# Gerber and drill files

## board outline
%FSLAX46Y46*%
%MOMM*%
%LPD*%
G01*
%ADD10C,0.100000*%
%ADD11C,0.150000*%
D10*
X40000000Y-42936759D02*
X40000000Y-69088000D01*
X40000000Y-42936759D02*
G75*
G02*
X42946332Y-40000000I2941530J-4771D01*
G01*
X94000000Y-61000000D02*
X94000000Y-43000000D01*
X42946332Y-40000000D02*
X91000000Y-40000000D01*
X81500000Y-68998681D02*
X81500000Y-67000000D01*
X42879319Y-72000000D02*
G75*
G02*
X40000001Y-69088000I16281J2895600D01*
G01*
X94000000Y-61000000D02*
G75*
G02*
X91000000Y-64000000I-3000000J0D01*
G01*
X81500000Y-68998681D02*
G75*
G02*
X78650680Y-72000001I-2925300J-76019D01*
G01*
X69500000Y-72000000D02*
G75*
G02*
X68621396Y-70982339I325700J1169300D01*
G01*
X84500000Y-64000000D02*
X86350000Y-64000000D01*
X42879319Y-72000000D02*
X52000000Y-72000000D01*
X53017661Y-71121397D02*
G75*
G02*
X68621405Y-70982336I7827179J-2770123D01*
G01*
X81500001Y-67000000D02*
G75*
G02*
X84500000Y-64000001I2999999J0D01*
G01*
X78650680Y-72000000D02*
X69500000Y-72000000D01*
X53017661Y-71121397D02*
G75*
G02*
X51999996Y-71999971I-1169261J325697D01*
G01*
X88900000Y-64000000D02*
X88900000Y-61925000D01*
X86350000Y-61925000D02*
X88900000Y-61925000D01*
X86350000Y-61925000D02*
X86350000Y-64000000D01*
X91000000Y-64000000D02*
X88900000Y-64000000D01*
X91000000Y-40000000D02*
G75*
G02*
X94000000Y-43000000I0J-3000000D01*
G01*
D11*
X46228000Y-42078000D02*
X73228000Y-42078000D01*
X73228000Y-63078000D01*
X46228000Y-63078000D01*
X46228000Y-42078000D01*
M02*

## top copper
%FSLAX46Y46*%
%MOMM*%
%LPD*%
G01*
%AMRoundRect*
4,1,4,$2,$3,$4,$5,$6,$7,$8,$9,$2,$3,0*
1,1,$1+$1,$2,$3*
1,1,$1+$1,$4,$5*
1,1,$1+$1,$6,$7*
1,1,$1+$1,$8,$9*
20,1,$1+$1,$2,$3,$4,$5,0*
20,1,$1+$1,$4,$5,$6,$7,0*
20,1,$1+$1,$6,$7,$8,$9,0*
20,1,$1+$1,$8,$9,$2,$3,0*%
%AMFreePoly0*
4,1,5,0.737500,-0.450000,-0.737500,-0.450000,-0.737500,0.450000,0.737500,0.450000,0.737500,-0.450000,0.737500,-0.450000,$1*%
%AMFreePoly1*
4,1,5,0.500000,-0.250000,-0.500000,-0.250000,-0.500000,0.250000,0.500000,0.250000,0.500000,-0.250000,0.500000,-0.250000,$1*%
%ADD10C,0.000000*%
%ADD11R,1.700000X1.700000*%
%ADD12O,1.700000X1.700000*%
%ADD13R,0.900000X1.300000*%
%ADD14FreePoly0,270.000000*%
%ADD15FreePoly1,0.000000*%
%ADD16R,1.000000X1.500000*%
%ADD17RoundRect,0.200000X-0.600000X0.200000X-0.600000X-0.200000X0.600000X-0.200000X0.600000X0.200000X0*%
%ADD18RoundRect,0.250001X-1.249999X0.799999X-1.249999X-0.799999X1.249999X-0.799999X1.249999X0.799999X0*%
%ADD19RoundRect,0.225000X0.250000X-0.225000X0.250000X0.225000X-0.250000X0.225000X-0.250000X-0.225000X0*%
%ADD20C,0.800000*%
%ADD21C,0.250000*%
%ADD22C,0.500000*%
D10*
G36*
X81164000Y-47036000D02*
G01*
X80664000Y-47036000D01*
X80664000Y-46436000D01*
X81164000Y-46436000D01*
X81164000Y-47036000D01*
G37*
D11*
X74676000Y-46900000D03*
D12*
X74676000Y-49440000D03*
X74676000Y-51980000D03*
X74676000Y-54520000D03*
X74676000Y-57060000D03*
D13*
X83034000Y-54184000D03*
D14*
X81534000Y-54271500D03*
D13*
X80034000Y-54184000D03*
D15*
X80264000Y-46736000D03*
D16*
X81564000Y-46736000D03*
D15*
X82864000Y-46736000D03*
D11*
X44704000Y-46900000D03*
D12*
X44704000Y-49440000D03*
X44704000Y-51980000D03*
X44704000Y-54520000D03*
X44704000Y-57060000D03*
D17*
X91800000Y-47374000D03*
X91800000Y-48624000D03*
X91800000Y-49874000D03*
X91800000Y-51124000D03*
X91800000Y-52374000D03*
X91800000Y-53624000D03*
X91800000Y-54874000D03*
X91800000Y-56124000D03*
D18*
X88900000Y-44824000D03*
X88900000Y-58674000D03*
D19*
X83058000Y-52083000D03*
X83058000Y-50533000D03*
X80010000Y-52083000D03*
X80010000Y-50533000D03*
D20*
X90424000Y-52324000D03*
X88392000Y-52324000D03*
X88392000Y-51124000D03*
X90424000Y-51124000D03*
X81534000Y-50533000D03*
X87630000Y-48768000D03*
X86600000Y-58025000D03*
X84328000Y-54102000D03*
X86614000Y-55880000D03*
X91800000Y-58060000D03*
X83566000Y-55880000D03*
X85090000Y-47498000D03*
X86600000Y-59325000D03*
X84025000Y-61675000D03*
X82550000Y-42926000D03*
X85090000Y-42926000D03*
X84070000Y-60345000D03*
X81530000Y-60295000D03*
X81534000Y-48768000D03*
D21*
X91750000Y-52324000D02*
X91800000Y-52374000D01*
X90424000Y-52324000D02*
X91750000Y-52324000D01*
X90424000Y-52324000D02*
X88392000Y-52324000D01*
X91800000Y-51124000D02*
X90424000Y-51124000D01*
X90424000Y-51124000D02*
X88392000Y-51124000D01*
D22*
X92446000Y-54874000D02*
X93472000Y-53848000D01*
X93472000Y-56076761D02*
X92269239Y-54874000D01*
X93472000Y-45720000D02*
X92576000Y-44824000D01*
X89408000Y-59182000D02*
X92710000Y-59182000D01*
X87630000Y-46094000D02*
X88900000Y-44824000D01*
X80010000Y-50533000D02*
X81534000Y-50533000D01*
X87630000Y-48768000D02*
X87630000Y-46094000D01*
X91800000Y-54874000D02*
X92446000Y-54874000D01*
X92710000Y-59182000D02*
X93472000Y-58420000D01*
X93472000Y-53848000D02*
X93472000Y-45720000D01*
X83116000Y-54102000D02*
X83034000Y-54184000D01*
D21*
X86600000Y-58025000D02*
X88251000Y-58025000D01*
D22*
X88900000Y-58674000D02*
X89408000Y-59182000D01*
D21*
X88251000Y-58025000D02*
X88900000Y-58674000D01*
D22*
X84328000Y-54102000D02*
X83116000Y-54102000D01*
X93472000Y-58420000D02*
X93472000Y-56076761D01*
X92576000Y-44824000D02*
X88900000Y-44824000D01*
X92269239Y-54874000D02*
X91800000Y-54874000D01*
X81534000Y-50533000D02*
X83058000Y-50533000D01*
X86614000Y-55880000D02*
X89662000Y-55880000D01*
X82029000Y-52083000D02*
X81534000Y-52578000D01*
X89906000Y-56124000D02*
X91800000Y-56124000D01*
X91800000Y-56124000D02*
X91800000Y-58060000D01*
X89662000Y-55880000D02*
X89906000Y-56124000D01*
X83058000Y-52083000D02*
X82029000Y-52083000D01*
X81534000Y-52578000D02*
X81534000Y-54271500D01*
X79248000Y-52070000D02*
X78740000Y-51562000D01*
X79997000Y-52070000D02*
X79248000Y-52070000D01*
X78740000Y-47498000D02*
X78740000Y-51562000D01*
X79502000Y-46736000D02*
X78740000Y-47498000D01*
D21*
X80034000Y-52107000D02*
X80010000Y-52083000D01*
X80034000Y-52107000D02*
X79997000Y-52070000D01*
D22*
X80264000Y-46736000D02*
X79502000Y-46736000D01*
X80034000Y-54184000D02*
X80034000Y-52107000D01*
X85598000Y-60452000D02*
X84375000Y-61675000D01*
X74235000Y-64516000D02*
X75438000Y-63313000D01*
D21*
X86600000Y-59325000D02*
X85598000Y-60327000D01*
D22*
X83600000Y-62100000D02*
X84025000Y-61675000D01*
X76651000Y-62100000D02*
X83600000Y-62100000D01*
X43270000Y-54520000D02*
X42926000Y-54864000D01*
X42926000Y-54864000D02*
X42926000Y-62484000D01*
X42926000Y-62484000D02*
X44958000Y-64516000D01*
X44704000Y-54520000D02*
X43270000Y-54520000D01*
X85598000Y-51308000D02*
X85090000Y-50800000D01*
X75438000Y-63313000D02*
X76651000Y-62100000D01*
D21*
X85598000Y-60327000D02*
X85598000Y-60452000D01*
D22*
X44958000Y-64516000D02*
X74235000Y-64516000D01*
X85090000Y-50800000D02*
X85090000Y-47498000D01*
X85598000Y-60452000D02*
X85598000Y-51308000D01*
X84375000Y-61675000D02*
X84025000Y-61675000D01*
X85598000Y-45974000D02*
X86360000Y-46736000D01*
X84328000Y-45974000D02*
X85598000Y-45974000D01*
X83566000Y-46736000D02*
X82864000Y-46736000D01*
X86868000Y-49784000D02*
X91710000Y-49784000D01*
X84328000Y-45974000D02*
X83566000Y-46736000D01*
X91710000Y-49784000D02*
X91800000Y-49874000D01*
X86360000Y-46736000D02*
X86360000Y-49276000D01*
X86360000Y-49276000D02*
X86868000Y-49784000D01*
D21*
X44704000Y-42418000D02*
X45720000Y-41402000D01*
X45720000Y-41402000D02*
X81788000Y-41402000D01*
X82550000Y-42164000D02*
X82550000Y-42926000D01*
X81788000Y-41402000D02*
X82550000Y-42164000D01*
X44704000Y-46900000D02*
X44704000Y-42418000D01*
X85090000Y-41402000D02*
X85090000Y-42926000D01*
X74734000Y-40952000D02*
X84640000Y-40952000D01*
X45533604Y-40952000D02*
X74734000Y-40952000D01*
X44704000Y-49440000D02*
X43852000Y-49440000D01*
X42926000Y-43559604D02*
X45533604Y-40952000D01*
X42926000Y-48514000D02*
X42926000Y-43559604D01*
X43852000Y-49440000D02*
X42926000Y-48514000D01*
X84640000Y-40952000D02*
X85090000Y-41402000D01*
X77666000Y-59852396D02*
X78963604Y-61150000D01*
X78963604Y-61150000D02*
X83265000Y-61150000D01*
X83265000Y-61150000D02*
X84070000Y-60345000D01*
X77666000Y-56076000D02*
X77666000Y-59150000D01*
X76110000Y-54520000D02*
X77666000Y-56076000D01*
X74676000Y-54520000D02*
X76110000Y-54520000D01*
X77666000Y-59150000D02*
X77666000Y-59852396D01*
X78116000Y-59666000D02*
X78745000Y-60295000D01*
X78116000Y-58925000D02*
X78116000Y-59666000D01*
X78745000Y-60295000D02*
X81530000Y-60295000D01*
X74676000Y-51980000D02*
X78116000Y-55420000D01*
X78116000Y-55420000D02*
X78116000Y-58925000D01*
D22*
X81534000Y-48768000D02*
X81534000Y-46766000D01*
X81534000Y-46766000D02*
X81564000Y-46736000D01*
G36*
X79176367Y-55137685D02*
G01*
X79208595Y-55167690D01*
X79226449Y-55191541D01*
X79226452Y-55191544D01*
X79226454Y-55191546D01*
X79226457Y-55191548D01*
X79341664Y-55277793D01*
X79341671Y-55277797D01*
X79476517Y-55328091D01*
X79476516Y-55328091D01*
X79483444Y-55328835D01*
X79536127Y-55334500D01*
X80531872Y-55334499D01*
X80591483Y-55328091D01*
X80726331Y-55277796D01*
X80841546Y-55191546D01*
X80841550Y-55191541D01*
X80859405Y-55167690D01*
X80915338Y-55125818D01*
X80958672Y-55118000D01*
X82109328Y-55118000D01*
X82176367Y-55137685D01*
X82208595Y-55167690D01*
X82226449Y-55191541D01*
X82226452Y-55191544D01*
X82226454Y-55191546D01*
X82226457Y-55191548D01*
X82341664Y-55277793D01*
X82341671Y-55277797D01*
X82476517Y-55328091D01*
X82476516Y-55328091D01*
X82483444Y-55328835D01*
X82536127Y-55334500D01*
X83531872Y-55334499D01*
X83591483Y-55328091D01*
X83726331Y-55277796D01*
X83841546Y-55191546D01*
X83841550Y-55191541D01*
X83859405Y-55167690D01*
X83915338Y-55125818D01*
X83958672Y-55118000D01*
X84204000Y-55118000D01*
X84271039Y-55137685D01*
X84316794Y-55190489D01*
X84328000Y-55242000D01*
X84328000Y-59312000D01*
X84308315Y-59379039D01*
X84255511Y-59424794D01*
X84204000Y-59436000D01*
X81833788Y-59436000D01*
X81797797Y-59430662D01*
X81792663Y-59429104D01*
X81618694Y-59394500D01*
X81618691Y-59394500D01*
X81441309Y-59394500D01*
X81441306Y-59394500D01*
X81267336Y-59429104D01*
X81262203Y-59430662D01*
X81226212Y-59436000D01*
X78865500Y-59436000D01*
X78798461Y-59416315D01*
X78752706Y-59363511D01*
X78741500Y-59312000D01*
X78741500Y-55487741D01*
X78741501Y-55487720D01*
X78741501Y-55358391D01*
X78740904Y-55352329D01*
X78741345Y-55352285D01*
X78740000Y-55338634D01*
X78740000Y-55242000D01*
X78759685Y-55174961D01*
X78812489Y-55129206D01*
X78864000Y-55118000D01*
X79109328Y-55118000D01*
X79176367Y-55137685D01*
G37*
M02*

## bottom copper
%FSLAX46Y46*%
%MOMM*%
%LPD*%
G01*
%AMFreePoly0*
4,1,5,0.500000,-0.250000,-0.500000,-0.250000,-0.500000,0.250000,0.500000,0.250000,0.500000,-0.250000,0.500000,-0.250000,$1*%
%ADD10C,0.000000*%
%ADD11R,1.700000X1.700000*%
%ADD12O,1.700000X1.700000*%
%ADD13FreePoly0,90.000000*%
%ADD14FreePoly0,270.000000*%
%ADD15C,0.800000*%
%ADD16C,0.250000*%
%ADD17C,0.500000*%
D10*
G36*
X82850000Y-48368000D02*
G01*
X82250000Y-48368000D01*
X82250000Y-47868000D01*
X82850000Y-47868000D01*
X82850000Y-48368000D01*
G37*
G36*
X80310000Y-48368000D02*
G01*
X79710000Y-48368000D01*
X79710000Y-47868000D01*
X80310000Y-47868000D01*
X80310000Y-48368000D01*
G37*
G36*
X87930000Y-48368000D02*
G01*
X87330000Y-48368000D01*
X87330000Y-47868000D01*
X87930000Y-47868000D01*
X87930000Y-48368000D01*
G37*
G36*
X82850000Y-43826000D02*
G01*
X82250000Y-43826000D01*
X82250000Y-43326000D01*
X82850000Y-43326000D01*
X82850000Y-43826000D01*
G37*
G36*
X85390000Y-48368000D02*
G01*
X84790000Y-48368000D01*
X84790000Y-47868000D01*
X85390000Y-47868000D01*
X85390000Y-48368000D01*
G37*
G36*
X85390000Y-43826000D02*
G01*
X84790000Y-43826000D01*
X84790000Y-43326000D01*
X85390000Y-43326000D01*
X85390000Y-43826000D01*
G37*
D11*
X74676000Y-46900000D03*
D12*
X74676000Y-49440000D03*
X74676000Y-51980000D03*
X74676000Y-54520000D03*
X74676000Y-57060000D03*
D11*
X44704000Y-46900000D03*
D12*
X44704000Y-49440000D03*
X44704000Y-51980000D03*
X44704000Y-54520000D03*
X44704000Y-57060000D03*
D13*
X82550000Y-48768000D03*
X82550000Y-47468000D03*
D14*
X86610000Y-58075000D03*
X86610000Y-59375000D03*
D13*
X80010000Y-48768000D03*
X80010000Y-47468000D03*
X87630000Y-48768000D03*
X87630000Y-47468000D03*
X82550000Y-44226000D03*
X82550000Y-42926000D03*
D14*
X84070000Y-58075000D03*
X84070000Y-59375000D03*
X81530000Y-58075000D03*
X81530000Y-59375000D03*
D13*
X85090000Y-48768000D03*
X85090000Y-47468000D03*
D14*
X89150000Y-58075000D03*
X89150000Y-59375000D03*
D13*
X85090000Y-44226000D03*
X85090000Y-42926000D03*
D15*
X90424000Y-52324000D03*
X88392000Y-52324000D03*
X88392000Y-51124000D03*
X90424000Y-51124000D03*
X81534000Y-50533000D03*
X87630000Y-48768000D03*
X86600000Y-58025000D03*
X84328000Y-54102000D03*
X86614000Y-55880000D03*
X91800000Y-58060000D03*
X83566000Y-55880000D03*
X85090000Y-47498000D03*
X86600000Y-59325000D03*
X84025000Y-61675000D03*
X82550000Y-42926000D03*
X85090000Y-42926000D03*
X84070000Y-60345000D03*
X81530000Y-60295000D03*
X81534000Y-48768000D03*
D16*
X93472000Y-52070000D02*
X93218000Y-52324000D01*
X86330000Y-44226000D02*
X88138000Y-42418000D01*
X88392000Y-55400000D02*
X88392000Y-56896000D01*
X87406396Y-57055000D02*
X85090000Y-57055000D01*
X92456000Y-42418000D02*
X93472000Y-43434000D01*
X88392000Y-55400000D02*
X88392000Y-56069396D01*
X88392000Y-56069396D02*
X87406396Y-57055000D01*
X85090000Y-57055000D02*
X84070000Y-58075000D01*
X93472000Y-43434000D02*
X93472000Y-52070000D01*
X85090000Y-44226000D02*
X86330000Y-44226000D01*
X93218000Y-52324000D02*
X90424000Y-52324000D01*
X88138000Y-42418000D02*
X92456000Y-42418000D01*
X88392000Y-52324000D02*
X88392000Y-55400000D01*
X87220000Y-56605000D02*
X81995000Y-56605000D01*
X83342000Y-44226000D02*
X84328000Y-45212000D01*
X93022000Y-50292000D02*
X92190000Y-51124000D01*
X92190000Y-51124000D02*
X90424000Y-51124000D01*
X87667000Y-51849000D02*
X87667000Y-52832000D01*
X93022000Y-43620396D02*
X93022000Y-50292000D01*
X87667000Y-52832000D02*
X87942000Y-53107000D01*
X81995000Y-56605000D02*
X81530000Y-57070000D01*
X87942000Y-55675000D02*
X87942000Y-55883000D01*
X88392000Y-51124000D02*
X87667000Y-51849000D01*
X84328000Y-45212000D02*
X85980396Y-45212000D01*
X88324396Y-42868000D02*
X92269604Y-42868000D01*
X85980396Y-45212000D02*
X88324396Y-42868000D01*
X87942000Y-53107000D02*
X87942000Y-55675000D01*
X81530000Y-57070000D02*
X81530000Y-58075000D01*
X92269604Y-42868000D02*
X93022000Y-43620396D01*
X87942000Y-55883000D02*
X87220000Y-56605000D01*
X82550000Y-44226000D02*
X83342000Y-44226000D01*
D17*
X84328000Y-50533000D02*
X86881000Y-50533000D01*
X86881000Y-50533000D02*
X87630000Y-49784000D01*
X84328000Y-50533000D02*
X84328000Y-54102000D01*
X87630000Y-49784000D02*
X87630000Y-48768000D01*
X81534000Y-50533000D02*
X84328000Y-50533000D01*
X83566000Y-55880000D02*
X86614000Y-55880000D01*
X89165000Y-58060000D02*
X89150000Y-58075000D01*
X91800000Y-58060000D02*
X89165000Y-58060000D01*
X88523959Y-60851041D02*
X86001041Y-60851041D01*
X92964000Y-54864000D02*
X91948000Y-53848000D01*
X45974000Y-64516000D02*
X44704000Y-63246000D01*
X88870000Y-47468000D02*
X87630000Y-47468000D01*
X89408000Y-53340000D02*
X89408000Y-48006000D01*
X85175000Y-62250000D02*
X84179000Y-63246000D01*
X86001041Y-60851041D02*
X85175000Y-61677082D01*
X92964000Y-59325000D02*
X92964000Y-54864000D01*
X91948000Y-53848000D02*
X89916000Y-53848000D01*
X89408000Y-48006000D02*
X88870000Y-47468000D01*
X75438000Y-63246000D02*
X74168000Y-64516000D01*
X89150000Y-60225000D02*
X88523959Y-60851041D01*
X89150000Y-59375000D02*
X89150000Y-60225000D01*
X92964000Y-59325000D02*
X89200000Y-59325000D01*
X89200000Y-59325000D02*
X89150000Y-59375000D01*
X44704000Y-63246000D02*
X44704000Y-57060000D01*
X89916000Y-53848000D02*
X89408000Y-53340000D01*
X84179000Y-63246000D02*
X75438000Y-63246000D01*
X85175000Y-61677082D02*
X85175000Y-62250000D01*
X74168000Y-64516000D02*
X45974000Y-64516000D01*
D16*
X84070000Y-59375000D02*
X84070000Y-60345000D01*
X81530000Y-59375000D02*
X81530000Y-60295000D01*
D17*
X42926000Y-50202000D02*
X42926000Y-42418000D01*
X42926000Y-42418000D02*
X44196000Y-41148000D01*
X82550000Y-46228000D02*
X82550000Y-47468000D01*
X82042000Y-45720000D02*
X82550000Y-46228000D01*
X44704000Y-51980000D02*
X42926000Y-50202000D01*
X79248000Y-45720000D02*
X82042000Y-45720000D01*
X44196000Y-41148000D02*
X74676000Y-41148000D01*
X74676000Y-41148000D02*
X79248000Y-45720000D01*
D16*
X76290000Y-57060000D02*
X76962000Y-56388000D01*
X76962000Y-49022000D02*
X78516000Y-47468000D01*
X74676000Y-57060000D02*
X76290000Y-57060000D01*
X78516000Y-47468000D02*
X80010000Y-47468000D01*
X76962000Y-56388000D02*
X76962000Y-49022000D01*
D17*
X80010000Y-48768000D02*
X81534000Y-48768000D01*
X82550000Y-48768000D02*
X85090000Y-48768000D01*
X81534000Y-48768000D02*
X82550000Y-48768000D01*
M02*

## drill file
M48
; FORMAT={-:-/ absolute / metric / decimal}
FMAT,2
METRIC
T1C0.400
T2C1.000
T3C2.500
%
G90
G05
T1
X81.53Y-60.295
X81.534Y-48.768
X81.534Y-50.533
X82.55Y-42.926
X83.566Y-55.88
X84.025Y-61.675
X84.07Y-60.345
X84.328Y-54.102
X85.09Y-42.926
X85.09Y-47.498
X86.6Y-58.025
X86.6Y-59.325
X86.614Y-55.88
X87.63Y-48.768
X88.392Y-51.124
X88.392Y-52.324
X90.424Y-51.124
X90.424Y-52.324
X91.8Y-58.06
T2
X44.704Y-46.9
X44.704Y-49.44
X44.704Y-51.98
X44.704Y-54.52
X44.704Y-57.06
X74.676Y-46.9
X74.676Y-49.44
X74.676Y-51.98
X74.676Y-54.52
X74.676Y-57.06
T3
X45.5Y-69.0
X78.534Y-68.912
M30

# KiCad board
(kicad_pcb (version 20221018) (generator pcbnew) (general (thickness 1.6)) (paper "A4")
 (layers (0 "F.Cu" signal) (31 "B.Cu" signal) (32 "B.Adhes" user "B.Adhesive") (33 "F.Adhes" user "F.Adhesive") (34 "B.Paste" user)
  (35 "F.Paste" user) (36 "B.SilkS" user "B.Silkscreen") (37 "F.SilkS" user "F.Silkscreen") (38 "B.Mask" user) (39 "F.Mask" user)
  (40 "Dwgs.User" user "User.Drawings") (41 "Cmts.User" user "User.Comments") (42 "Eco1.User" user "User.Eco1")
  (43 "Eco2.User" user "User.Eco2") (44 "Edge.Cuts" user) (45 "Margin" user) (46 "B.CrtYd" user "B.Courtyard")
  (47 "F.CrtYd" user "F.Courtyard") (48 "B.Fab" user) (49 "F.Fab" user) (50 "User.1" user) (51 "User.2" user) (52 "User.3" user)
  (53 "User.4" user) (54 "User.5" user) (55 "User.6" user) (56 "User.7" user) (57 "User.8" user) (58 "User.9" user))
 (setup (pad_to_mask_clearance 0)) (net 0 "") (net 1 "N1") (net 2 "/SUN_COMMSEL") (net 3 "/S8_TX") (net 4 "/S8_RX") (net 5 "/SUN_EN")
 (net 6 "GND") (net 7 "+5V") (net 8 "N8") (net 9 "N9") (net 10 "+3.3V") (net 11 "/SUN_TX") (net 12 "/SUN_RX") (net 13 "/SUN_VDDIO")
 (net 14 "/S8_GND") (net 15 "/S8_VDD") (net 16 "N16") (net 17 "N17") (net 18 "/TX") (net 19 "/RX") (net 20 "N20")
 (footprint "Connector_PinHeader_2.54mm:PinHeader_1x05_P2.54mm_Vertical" (layer "F.Cu") (at 74.676 46.9)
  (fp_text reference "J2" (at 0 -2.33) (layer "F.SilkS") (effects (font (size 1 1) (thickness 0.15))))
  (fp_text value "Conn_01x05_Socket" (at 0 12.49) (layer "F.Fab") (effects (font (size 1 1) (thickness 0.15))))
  (pad "1" thru_hole rect (at 0 0) (size 1.7 1.7) (drill 1) (layers "*.Cu" "*.Mask") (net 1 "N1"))
  (pad "2" thru_hole oval (at 0 2.54) (size 1.7 1.7) (drill 1) (layers "*.Cu" "*.Mask") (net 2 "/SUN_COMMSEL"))
  (pad "3" thru_hole oval (at 0 5.08) (size 1.7 1.7) (drill 1) (layers "*.Cu" "*.Mask") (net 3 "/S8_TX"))
  (pad "4" thru_hole oval (at 0 7.62) (size 1.7 1.7) (drill 1) (layers "*.Cu" "*.Mask") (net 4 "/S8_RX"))
  (pad "5" thru_hole oval (at 0 10.16) (size 1.7 1.7) (drill 1) (layers "*.Cu" "*.Mask") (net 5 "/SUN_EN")))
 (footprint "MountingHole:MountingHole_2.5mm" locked (layer "F.Cu") (at 45.466 69.088)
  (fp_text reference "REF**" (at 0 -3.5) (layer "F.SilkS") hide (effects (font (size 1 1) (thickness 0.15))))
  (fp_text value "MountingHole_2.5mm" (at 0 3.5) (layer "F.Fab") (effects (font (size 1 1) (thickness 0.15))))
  (pad "" np_thru_hole circle locked (at 0.034 -0.088) (size 2.5 2.5) (drill 2.5) (layers "F&B.Cu" "*.Mask")))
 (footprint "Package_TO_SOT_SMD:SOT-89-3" (layer "F.Cu") (at 81.534 56.134 -90)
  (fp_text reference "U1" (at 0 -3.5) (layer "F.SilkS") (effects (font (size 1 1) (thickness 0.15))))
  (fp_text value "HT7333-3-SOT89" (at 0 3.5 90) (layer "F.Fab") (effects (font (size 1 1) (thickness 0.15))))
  (pad "1" smd rect (at -1.95 -1.5 270) (size 1.3 0.9) (layers "F.Cu" "F.Paste" "F.Mask") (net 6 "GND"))
  (pad "2" smd custom (at -1.8625 0 270) (size 1.475 0.9) (layers "F.Cu" "F.Paste" "F.Mask") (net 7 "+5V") (zone_connect 2)
   (thermal_bridge_angle 45) (options (clearance outline) (anchor rect)) (primitives))
  (pad "3" smd rect (at -1.95 1.5 270) (size 1.3 0.9) (layers "F.Cu" "F.Paste" "F.Mask") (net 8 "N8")))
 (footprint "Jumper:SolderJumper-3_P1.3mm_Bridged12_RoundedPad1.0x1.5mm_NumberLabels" (layer "F.Cu") (at 81.564 46.736)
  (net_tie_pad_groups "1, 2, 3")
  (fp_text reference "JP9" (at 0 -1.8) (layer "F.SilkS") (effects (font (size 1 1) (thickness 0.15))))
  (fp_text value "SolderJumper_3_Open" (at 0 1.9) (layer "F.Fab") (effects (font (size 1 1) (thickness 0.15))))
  (fp_poly (pts (xy -0.9 -0.3) (xy -0.4 -0.3) (xy -0.4 0.3) (xy -0.9 0.3)) (stroke (width 0) (type solid)) (fill solid) (layer "F.Cu"))
  (pad "1" smd custom (at -1.3 0) (size 1 0.5) (layers "F.Cu" "F.Mask") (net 8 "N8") (zone_connect 2) (thermal_bridge_angle 45)
   (options (clearance outline) (anchor rect)) (primitives))
  (pad "2" smd rect (at 0 0) (size 1 1.5) (layers "F.Cu" "F.Mask") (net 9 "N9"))
  (pad "3" smd custom (at 1.3 0) (size 1 0.5) (layers "F.Cu" "F.Mask") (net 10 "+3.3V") (zone_connect 2) (thermal_bridge_angle 45)
   (options (clearance outline) (anchor rect)) (primitives)))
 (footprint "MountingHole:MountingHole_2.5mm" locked (layer "F.Cu") (at 78.5 69)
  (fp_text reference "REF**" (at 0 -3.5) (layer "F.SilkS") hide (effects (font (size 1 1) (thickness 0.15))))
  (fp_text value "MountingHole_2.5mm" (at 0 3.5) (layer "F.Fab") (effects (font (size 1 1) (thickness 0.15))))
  (pad "" np_thru_hole circle locked (at 0.034 -0.088) (size 2.5 2.5) (drill 2.5) (layers "F&B.Cu" "*.Mask")))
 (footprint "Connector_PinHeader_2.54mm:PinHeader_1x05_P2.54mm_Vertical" (layer "F.Cu") (at 44.704 46.9)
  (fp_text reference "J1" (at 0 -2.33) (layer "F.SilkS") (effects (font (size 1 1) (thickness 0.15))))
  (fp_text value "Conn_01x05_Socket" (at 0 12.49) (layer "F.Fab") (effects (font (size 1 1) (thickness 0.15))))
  (pad "1" thru_hole rect (at 0 0) (size 1.7 1.7) (drill 1) (layers "*.Cu" "*.Mask") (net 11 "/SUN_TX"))
  (pad "2" thru_hole oval (at 0 2.54) (size 1.7 1.7) (drill 1) (layers "*.Cu" "*.Mask") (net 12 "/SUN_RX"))
  (pad "3" thru_hole oval (at 0 5.08) (size 1.7 1.7) (drill 1) (layers "*.Cu" "*.Mask") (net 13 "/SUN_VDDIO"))
  (pad "4" thru_hole oval (at 0 7.62) (size 1.7 1.7) (drill 1) (layers "*.Cu" "*.Mask") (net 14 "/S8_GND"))
  (pad "5" thru_hole oval (at 0 10.16) (size 1.7 1.7) (drill 1) (layers "*.Cu" "*.Mask") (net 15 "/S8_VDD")))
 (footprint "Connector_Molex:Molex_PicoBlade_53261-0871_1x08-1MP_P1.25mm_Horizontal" (layer "F.Cu") (at 89.4 51.749 -90)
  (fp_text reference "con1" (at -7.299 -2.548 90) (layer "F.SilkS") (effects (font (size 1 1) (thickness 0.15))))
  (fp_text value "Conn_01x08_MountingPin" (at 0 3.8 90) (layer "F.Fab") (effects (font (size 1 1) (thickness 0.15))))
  (pad "1" smd roundrect (at -4.375 -2.4 270) (size 0.8 1.6) (layers "F.Cu" "F.Paste" "F.Mask") (roundrect_rratio 0.25) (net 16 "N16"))
  (pad "2" smd roundrect (at -3.125 -2.4 270) (size 0.8 1.6) (layers "F.Cu" "F.Paste" "F.Mask") (roundrect_rratio 0.25) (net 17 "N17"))
  (pad "3" smd roundrect (at -1.875 -2.4 270) (size 0.8 1.6) (layers "F.Cu" "F.Paste" "F.Mask") (roundrect_rratio 0.25) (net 10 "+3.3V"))
  (pad "4" smd roundrect (at -0.625 -2.4 270) (size 0.8 1.6) (layers "F.Cu" "F.Paste" "F.Mask") (roundrect_rratio 0.25) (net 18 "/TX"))
  (pad "5" smd roundrect (at 0.625 -2.4 270) (size 0.8 1.6) (layers "F.Cu" "F.Paste" "F.Mask") (roundrect_rratio 0.25) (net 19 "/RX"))
  (pad "6" smd roundrect (at 1.875 -2.4 270) (size 0.8 1.6) (layers "F.Cu" "F.Paste" "F.Mask") (roundrect_rratio 0.25) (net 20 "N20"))
  (pad "7" smd roundrect (at 3.125 -2.4 270) (size 0.8 1.6) (layers "F.Cu" "F.Paste" "F.Mask") (roundrect_rratio 0.25) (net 6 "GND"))
  (pad "8" smd roundrect (at 4.375 -2.4 270) (size 0.8 1.6) (layers "F.Cu" "F.Paste" "F.Mask") (roundrect_rratio 0.25) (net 7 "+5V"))
  (pad "MP" smd roundrect (at -6.925 0.5 270) (size 2.1 3) (layers "F.Cu" "F.Paste" "F.Mask") (roundrect_rratio 0.1190480952) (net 6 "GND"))
  (pad "MP" smd roundrect (at 6.925 0.5 270) (size 2.1 3) (layers "F.Cu" "F.Paste" "F.Mask") (roundrect_rratio 0.1190480952) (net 6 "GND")))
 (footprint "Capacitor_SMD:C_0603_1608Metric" (layer "F.Cu") (at 83.058 51.308 90)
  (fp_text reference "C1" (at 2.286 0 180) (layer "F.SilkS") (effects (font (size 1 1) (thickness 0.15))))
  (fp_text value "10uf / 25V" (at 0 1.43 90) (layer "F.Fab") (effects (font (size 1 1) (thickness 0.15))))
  (pad "1" smd roundrect (at -0.775 0 90) (size 0.9 0.95) (layers "F.Cu" "F.Paste" "F.Mask") (roundrect_rratio 0.25) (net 7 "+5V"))
  (pad "2" smd roundrect (at 0.775 0 90) (size 0.9 0.95) (layers "F.Cu" "F.Paste" "F.Mask") (roundrect_rratio 0.25) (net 6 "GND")))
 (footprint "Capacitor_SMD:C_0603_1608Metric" (layer "F.Cu") (at 80.01 51.308 90)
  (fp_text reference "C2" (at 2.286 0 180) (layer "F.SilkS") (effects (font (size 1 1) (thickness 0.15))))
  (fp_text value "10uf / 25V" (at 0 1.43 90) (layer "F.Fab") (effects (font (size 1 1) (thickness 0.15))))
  (pad "1" smd roundrect (at -0.775 0 90) (size 0.9 0.95) (layers "F.Cu" "F.Paste" "F.Mask") (roundrect_rratio 0.25) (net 8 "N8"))
  (pad "2" smd roundrect (at 0.775 0 90) (size 0.9 0.95) (layers "F.Cu" "F.Paste" "F.Mask") (roundrect_rratio 0.25) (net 6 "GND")))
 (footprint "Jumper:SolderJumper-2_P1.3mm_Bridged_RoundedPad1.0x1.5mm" (layer "B.Cu") (at 82.55 48.118 90) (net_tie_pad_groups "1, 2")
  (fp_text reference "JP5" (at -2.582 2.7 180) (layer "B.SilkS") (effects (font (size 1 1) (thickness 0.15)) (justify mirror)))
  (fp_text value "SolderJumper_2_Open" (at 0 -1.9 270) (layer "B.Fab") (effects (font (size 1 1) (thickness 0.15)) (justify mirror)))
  (fp_poly (pts (xy 0.25 0.3) (xy -0.25 0.3) (xy -0.25 -0.3) (xy 0.25 -0.3)) (stroke (width 0) (type solid)) (fill solid) (layer "B.Cu"))
  (pad "1" smd custom (at -0.65 0 90) (size 1 0.5) (layers "B.Cu" "B.Mask") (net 9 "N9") (zone_connect 2) (thermal_bridge_angle 45)
   (options (clearance outline) (anchor rect)) (primitives))
  (pad "2" smd custom (at 0.65 0 90) (size 1 0.5) (layers "B.Cu" "B.Mask") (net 13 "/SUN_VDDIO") (zone_connect 2) (thermal_bridge_angle 45)
   (options (clearance outline) (anchor rect)) (primitives)))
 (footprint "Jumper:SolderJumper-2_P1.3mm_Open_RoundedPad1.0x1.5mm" (layer "B.Cu") (at 86.61 58.725 -90)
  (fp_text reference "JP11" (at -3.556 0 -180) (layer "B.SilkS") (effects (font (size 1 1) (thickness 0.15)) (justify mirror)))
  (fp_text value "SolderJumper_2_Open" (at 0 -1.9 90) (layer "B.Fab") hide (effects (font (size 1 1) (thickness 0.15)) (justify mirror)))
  (pad "1" smd custom (at -0.65 0 270) (size 1 0.5) (layers "B.Cu" "B.Mask") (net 6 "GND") (zone_connect 2) (thermal_bridge_angle 45)
   (options (clearance outline) (anchor rect)) (primitives))
  (pad "2" smd custom (at 0.65 0 270) (size 1 0.5) (layers "B.Cu" "B.Mask") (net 14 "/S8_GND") (zone_connect 2) (thermal_bridge_angle 45)
   (options (clearance outline) (anchor rect)) (primitives)))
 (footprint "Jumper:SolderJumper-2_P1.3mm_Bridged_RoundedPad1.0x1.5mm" (layer "B.Cu") (at 80.01 48.118 90) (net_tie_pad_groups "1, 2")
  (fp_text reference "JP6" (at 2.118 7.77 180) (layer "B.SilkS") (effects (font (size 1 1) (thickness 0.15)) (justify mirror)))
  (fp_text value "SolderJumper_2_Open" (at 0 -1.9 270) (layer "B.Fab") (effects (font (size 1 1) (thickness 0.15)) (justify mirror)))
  (fp_poly (pts (xy 0.25 0.3) (xy -0.25 0.3) (xy -0.25 -0.3) (xy 0.25 -0.3)) (stroke (width 0) (type solid)) (fill solid) (layer "B.Cu"))
  (pad "1" smd custom (at -0.65 0 90) (size 1 0.5) (layers "B.Cu" "B.Mask") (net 9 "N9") (zone_connect 2) (thermal_bridge_angle 45)
   (options (clearance outline) (anchor rect)) (primitives))
  (pad "2" smd custom (at 0.65 0 90) (size 1 0.5) (layers "B.Cu" "B.Mask") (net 5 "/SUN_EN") (zone_connect 2) (thermal_bridge_angle 45)
   (options (clearance outline) (anchor rect)) (primitives)))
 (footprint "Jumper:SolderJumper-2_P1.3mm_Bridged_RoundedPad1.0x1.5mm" (layer "B.Cu") (at 87.63 48.118 90) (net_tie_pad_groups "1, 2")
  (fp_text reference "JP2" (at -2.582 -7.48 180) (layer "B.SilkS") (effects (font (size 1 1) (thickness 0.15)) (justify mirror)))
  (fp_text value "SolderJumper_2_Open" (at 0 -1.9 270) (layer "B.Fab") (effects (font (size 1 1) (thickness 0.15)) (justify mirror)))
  (fp_poly (pts (xy 0.25 0.3) (xy -0.25 0.3) (xy -0.25 -0.3) (xy 0.25 -0.3)) (stroke (width 0) (type solid)) (fill solid) (layer "B.Cu"))
  (pad "1" smd custom (at -0.65 0 90) (size 1 0.5) (layers "B.Cu" "B.Mask") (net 6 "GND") (zone_connect 2) (thermal_bridge_angle 45)
   (options (clearance outline) (anchor rect)) (primitives))
  (pad "2" smd custom (at 0.65 0 90) (size 1 0.5) (layers "B.Cu" "B.Mask") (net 15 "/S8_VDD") (zone_connect 2) (thermal_bridge_angle 45)
   (options (clearance outline) (anchor rect)) (primitives)))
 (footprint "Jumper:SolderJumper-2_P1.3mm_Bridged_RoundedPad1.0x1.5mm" (layer "B.Cu") (at 82.55 43.576 90) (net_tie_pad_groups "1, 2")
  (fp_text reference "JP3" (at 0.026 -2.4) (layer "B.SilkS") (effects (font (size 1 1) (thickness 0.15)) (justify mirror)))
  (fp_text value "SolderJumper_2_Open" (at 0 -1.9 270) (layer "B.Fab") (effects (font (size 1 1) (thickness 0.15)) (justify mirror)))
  (fp_poly (pts (xy 0.25 0.3) (xy -0.25 0.3) (xy -0.25 -0.3) (xy 0.25 -0.3)) (stroke (width 0) (type solid)) (fill solid) (layer "B.Cu"))
  (pad "1" smd custom (at -0.65 0 90) (size 1 0.5) (layers "B.Cu" "B.Mask") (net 18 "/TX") (zone_connect 2) (thermal_bridge_angle 45)
   (options (clearance outline) (anchor rect)) (primitives))
  (pad "2" smd custom (at 0.65 0 90) (size 1 0.5) (layers "B.Cu" "B.Mask") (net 11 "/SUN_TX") (zone_connect 2) (thermal_bridge_angle 45)
   (options (clearance outline) (anchor rect)) (primitives)))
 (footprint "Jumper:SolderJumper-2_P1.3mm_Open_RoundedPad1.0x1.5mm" (layer "B.Cu") (at 84.07 58.725 -90)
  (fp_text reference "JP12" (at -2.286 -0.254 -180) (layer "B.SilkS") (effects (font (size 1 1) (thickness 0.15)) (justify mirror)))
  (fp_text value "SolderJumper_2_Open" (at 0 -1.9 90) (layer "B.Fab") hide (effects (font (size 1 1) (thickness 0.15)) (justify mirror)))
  (pad "1" smd custom (at -0.65 0 270) (size 1 0.5) (layers "B.Cu" "B.Mask") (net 19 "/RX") (zone_connect 2) (thermal_bridge_angle 45)
   (options (clearance outline) (anchor rect)) (primitives))
  (pad "2" smd custom (at 0.65 0 270) (size 1 0.5) (layers "B.Cu" "B.Mask") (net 4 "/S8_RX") (zone_connect 2) (thermal_bridge_angle 45)
   (options (clearance outline) (anchor rect)) (primitives)))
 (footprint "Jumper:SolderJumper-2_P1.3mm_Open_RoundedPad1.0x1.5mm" (layer "B.Cu") (at 81.53 58.725 -90)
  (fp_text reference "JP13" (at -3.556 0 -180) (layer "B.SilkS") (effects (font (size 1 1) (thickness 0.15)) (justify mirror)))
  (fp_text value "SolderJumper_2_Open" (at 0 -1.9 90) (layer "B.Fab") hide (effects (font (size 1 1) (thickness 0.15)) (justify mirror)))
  (pad "1" smd custom (at -0.65 0 270) (size 1 0.5) (layers "B.Cu" "B.Mask") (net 18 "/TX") (zone_connect 2) (thermal_bridge_angle 45)
   (options (clearance outline) (anchor rect)) (primitives))
  (pad "2" smd custom (at 0.65 0 270) (size 1 0.5) (layers "B.Cu" "B.Mask") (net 3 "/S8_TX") (zone_connect 2) (thermal_bridge_angle 45)
   (options (clearance outline) (anchor rect)) (primitives)))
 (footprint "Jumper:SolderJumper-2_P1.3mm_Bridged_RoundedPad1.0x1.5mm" (layer "B.Cu") (at 85.09 48.118 90) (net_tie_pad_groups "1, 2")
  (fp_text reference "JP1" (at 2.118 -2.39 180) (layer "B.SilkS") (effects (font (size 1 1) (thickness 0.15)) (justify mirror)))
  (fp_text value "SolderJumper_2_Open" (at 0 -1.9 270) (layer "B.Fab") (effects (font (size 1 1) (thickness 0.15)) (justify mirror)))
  (fp_poly (pts (xy 0.25 0.3) (xy -0.25 0.3) (xy -0.25 -0.3) (xy 0.25 -0.3)) (stroke (width 0) (type solid)) (fill solid) (layer "B.Cu"))
  (pad "1" smd custom (at -0.65 0 90) (size 1 0.5) (layers "B.Cu" "B.Mask") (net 9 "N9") (zone_connect 2) (thermal_bridge_angle 45)
   (options (clearance outline) (anchor rect)) (primitives))
  (pad "2" smd custom (at 0.65 0 90) (size 1 0.5) (layers "B.Cu" "B.Mask") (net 14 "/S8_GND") (zone_connect 2) (thermal_bridge_angle 45)
   (options (clearance outline) (anchor rect)) (primitives)))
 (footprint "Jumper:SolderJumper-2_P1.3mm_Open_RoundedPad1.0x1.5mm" (layer "B.Cu") (at 89.15 58.725 -90)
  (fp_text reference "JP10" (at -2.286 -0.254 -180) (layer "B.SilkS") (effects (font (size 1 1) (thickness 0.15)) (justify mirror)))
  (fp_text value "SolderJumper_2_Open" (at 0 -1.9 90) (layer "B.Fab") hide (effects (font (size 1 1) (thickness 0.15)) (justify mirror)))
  (pad "1" smd custom (at -0.65 0 270) (size 1 0.5) (layers "B.Cu" "B.Mask") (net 7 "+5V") (zone_connect 2) (thermal_bridge_angle 45)
   (options (clearance outline) (anchor rect)) (primitives))
  (pad "2" smd custom (at 0.65 0 270) (size 1 0.5) (layers "B.Cu" "B.Mask") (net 15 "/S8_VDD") (zone_connect 2) (thermal_bridge_angle 45)
   (options (clearance outline) (anchor rect)) (primitives)))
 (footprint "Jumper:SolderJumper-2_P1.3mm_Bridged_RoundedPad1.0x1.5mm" (layer "B.Cu") (at 85.09 43.576 90) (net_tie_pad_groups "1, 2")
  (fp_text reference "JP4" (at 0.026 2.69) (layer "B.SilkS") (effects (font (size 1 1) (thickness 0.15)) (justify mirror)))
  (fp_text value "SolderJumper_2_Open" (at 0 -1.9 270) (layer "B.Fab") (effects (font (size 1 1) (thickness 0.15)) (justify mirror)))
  (fp_poly (pts (xy 0.25 0.3) (xy -0.25 0.3) (xy -0.25 -0.3) (xy 0.25 -0.3)) (stroke (width 0) (type solid)) (fill solid) (layer "B.Cu"))
  (pad "1" smd custom (at -0.65 0 90) (size 1 0.5) (layers "B.Cu" "B.Mask") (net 19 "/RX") (zone_connect 2) (thermal_bridge_angle 45)
   (options (clearance outline) (anchor rect)) (primitives))
  (pad "2" smd custom (at 0.65 0 90) (size 1 0.5) (layers "B.Cu" "B.Mask") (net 12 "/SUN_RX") (zone_connect 2) (thermal_bridge_angle 45)
   (options (clearance outline) (anchor rect)) (primitives)))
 (gr_line locked (start 40 42.936759) (end 40 69.088) (stroke (width 0.1) (type default)) (layer "Edge.Cuts"))
 (gr_arc locked (start 40 42.936759) (mid 40.864938 40.858169) (end 42.946332 40) (stroke (width 0.1) (type default)) (layer "Edge.Cuts"))
 (gr_line locked (start 94 61) (end 94 43) (stroke (width 0.1) (type default)) (layer "Edge.Cuts"))
 (gr_line locked (start 42.946332 40) (end 91 40) (stroke (width 0.1) (type default)) (layer "Edge.Cuts"))
 (gr_line locked (start 81.5 68.998681) (end 81.5 67) (stroke (width 0.1) (type default)) (layer "Edge.Cuts"))
 (gr_arc locked (start 42.879319 72) (mid 40.83656 71.140332) (end 40 69.088) (stroke (width 0.1) (type default)) (layer "Edge.Cuts"))
 (gr_arc locked (start 94 61) (mid 93.121321 63.121321) (end 91 64) (stroke (width 0.1) (type default)) (layer "Edge.Cuts"))
 (gr_arc locked (start 81.5 68.998681) (mid 80.696939 71.089459) (end 78.65068 72) (stroke (width 0.1) (type default)) (layer "Edge.Cuts"))
 (gr_arc locked (start 69.5 72) (mid 68.906927 71.623929) (end 68.621397 70.982339) (stroke (width 0.1) (type default)) (layer "Edge.Cuts"))
 (gr_line locked (start 84.5 64) (end 86.35 64) (stroke (width 0.1) (type default)) (layer "Edge.Cuts"))
 (gr_line locked (start 42.879319 72) (end 52 72) (stroke (width 0.1) (type default)) (layer "Edge.Cuts"))
 (gr_arc locked (start 53.017661 71.121397) (mid 60.770843 65.588942) (end 68.621397 70.982339) (stroke (width 0.1) (type default))
  (layer "Edge.Cuts"))
 (gr_arc locked (start 81.500001 67) (mid 82.37868 64.878681) (end 84.5 64) (stroke (width 0.1) (type default)) (layer "Edge.Cuts"))
 (gr_line locked (start 78.65068 72) (end 69.5 72) (stroke (width 0.1) (type default)) (layer "Edge.Cuts"))
 (gr_arc locked (start 53.017661 71.121397) (mid 52.64159 71.71447) (end 52 72) (stroke (width 0.1) (type default)) (layer "Edge.Cuts"))
 (gr_line locked (start 88.9 64) (end 88.9 61.925) (stroke (width 0.1) (type default)) (layer "Edge.Cuts"))
 (gr_line locked (start 86.35 61.925) (end 88.9 61.925) (stroke (width 0.1) (type default)) (layer "Edge.Cuts"))
 (gr_line locked (start 86.35 61.925) (end 86.35 64) (stroke (width 0.1) (type default)) (layer "Edge.Cuts"))
 (gr_line locked (start 91 64) (end 88.9 64) (stroke (width 0.1) (type default)) (layer "Edge.Cuts"))
 (gr_arc locked (start 91 40) (mid 93.121321 40.878679) (end 94 43) (stroke (width 0.1) (type default)) (layer "Edge.Cuts"))
 (gr_rect locked (start 46.228 42.078) (end 73.228 63.078) (stroke (width 0.15) (type default)) (fill none) (layer "Edge.Cuts"))
 (segment (start 91.75 52.324) (end 91.8 52.374) (width 0.25) (layer "F.Cu") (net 19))
 (segment (start 90.424 52.324) (end 91.75 52.324) (width 0.25) (layer "F.Cu") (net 19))
 (segment (start 90.424 52.324) (end 88.392 52.324) (width 0.25) (layer "F.Cu") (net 19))
 (via (at 90.424 52.324) (size 0.8) (drill 0.4) (layers "F.Cu" "B.Cu") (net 19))
 (via (at 88.392 52.324) (size 0.8) (drill 0.4) (layers "F.Cu" "B.Cu") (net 19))
 (segment (start 93.472 52.07) (end 93.218 52.324) (width 0.25) (layer "B.Cu") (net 19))
 (segment (start 86.33 44.226) (end 88.138 42.418) (width 0.25) (layer "B.Cu") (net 19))
 (segment (start 88.392 55.4) (end 88.392 56.896) (width 0.25) (layer "B.Cu") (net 19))
 (segment (start 87.406396 57.055) (end 85.09 57.055) (width 0.25) (layer "B.Cu") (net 19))
 (segment (start 92.456 42.418) (end 93.472 43.434) (width 0.25) (layer "B.Cu") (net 19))
 (segment (start 88.392 55.4) (end 88.392 56.069396) (width 0.25) (layer "B.Cu") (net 19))
 (segment (start 88.392 56.069396) (end 87.406396 57.055) (width 0.25) (layer "B.Cu") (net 19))
 (segment (start 85.09 57.055) (end 84.07 58.075) (width 0.25) (layer "B.Cu") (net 19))
 (segment (start 93.472 43.434) (end 93.472 52.07) (width 0.25) (layer "B.Cu") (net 19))
 (segment (start 85.09 44.226) (end 86.33 44.226) (width 0.25) (layer "B.Cu") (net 19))
 (segment (start 93.218 52.324) (end 90.424 52.324) (width 0.25) (layer "B.Cu") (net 19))
 (segment (start 88.138 42.418) (end 92.456 42.418) (width 0.25) (layer "B.Cu") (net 19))
 (segment (start 88.392 52.324) (end 88.392 55.4) (width 0.25) (layer "B.Cu") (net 19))
 (segment (start 91.8 51.124) (end 90.424 51.124) (width 0.25) (layer "F.Cu") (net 18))
 (segment (start 90.424 51.124) (end 88.392 51.124) (width 0.25) (layer "F.Cu") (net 18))
 (via (at 88.392 51.124) (size 0.8) (drill 0.4) (layers "F.Cu" "B.Cu") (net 18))
 (via (at 90.424 51.124) (size 0.8) (drill 0.4) (layers "F.Cu" "B.Cu") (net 18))
 (segment (start 87.22 56.605) (end 81.995 56.605) (width 0.25) (layer "B.Cu") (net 18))
 (segment (start 83.342 44.226) (end 84.328 45.212) (width 0.25) (layer "B.Cu") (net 18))
 (segment (start 93.022 50.292) (end 92.19 51.124) (width 0.25) (layer "B.Cu") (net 18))
 (segment (start 92.19 51.124) (end 90.424 51.124) (width 0.25) (layer "B.Cu") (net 18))
 (segment (start 87.667 51.849) (end 87.667 52.832) (width 0.25) (layer "B.Cu") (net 18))
 (segment (start 93.022 43.620396) (end 93.022 50.292) (width 0.25) (layer "B.Cu") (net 18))
 (segment (start 87.667 52.832) (end 87.942 53.107) (width 0.25) (layer "B.Cu") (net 18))
 (segment (start 81.995 56.605) (end 81.53 57.07) (width 0.25) (layer "B.Cu") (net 18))
 (segment (start 87.942 55.675) (end 87.942 55.883) (width 0.25) (layer "B.Cu") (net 18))
 (segment (start 88.392 51.124) (end 87.667 51.849) (width 0.25) (layer "B.Cu") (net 18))
 (segment (start 84.328 45.212) (end 85.980396 45.212) (width 0.25) (layer "B.Cu") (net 18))
 (segment (start 88.324396 42.868) (end 92.269604 42.868) (width 0.25) (layer "B.Cu") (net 18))
 (segment (start 85.980396 45.212) (end 88.324396 42.868) (width 0.25) (layer "B.Cu") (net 18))
 (segment (start 87.942 53.107) (end 87.942 55.675) (width 0.25) (layer "B.Cu") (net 18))
 (segment (start 81.53 57.07) (end 81.53 58.075) (width 0.25) (layer "B.Cu") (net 18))
 (segment (start 92.269604 42.868) (end 93.022 43.620396) (width 0.25) (layer "B.Cu") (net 18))
 (segment (start 87.942 55.883) (end 87.22 56.605) (width 0.25) (layer "B.Cu") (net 18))
 (segment (start 82.55 44.226) (end 83.342 44.226) (width 0.25) (layer "B.Cu") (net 18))
 (segment (start 92.446 54.874) (end 93.472 53.848) (width 0.5) (layer "F.Cu") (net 6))
 (segment (start 93.472 56.076761) (end 92.269239 54.874) (width 0.5) (layer "F.Cu") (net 6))
 (segment (start 93.472 45.72) (end 92.576 44.824) (width 0.5) (layer "F.Cu") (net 6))
 (segment (start 89.408 59.182) (end 92.71 59.182) (width 0.5) (layer "F.Cu") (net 6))
 (segment (start 87.63 46.094) (end 88.9 44.824) (width 0.5) (layer "F.Cu") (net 6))
 (segment (start 80.01 50.533) (end 81.534 50.533) (width 0.5) (layer "F.Cu") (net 6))
 (segment (start 87.63 48.768) (end 87.63 46.094) (width 0.5) (layer "F.Cu") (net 6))
 (segment (start 91.8 54.874) (end 92.446 54.874) (width 0.5) (layer "F.Cu") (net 6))
 (segment (start 92.71 59.182) (end 93.472 58.42) (width 0.5) (layer "F.Cu") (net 6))
 (segment (start 93.472 53.848) (end 93.472 45.72) (width 0.5) (layer "F.Cu") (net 6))
 (segment (start 83.116 54.102) (end 83.034 54.184) (width 0.5) (layer "F.Cu") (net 6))
 (segment (start 86.6 58.025) (end 88.251 58.025) (width 0.25) (layer "F.Cu") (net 6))
 (segment (start 88.9 58.674) (end 89.408 59.182) (width 0.5) (layer "F.Cu") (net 6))
 (segment (start 88.251 58.025) (end 88.9 58.674) (width 0.25) (layer "F.Cu") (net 6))
 (segment (start 84.328 54.102) (end 83.116 54.102) (width 0.5) (layer "F.Cu") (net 6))
 (segment (start 93.472 58.42) (end 93.472 56.076761) (width 0.5) (layer "F.Cu") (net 6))
 (segment (start 92.576 44.824) (end 88.9 44.824) (width 0.5) (layer "F.Cu") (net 6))
 (segment (start 92.269239 54.874) (end 91.8 54.874) (width 0.5) (layer "F.Cu") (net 6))
 (segment (start 81.534 50.533) (end 83.058 50.533) (width 0.5) (layer "F.Cu") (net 6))
 (via (at 81.534 50.533) (size 0.8) (drill 0.4) (layers "F.Cu" "B.Cu") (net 6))
 (via (at 87.63 48.768) (size 0.8) (drill 0.4) (layers "F.Cu" "B.Cu") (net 6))
 (via (at 86.6 58.025) (size 0.8) (drill 0.4) (layers "F.Cu" "B.Cu") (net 6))
 (via (at 84.328 54.102) (size 0.8) (drill 0.4) (layers "F.Cu" "B.Cu") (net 6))
 (segment (start 84.328 50.533) (end 86.881 50.533) (width 0.5) (layer "B.Cu") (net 6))
 (segment (start 86.881 50.533) (end 87.63 49.784) (width 0.5) (layer "B.Cu") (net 6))
 (segment (start 84.328 50.533) (end 84.328 54.102) (width 0.5) (layer "B.Cu") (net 6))
 (segment (start 87.63 49.784) (end 87.63 48.768) (width 0.5) (layer "B.Cu") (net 6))
 (segment (start 81.534 50.533) (end 84.328 50.533) (width 0.5) (layer "B.Cu") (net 6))
 (segment (start 86.614 55.88) (end 89.662 55.88) (width 0.5) (layer "F.Cu") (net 7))
 (segment (start 82.029 52.083) (end 81.534 52.578) (width 0.5) (layer "F.Cu") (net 7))
 (segment (start 89.906 56.124) (end 91.8 56.124) (width 0.5) (layer "F.Cu") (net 7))
 (segment (start 91.8 56.124) (end 91.8 58.06) (width 0.5) (layer "F.Cu") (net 7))
 (segment (start 89.662 55.88) (end 89.906 56.124) (width 0.5) (layer "F.Cu") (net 7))
 (segment (start 83.058 52.083) (end 82.029 52.083) (width 0.5) (layer "F.Cu") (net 7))
 (segment (start 81.534 52.578) (end 81.534 54.2715) (width 0.5) (layer "F.Cu") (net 7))
 (via (at 86.614 55.88) (size 0.8) (drill 0.4) (layers "F.Cu" "B.Cu") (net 7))
 (via (at 91.8 58.06) (size 0.8) (drill 0.4) (layers "F.Cu" "B.Cu") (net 7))
 (via (at 83.566 55.88) (size 0.8) (drill 0.4) (layers "F.Cu" "B.Cu") (free) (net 7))
 (segment (start 83.566 55.88) (end 86.614 55.88) (width 0.5) (layer "B.Cu") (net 7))
 (segment (start 89.165 58.06) (end 89.15 58.075) (width 0.5) (layer "B.Cu") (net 7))
 (segment (start 91.8 58.06) (end 89.165 58.06) (width 0.5) (layer "B.Cu") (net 7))
 (segment (start 79.248 52.07) (end 78.74 51.562) (width 0.5) (layer "F.Cu") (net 8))
 (segment (start 79.997 52.07) (end 79.248 52.07) (width 0.5) (layer "F.Cu") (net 8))
 (segment (start 78.74 47.498) (end 78.74 51.562) (width 0.5) (layer "F.Cu") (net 8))
 (segment (start 79.502 46.736) (end 78.74 47.498) (width 0.5) (layer "F.Cu") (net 8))
 (segment (start 80.034 52.107) (end 80.01 52.083) (width 0.25) (layer "F.Cu") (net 8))
 (segment (start 80.034 52.107) (end 79.997 52.07) (width 0.25) (layer "F.Cu") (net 8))
 (segment (start 80.264 46.736) (end 79.502 46.736) (width 0.5) (layer "F.Cu") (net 8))
 (segment (start 80.034 54.184) (end 80.034 52.107) (width 0.5) (layer "F.Cu") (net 8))
 (segment (start 88.523959 60.851041) (end 86.001041 60.851041) (width 0.5) (layer "B.Cu") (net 15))
 (segment (start 92.964 54.864) (end 91.948 53.848) (width 0.5) (layer "B.Cu") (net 15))
 (segment (start 45.974 64.516) (end 44.704 63.246) (width 0.5) (layer "B.Cu") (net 15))
 (segment (start 88.87 47.468) (end 87.63 47.468) (width 0.5) (layer "B.Cu") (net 15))
 (segment (start 89.408 53.34) (end 89.408 48.006) (width 0.5) (layer "B.Cu") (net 15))
 (segment (start 85.175 62.25) (end 84.179 63.246) (width 0.5) (layer "B.Cu") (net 15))
 (segment (start 86.001041 60.851041) (end 85.175 61.677082) (width 0.5) (layer "B.Cu") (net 15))
 (segment (start 92.964 59.325) (end 92.964 54.864) (width 0.5) (layer "B.Cu") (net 15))
 (segment (start 91.948 53.848) (end 89.916 53.848) (width 0.5) (layer "B.Cu") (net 15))
 (segment (start 89.408 48.006) (end 88.87 47.468) (width 0.5) (layer "B.Cu") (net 15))
 (segment (start 75.438 63.246) (end 74.168 64.516) (width 0.5) (layer "B.Cu") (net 15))
 (segment (start 89.15 60.225) (end 88.523959 60.851041) (width 0.5) (layer "B.Cu") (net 15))
 (segment (start 89.15 59.375) (end 89.15 60.225) (width 0.5) (layer "B.Cu") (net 15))
 (segment (start 92.964 59.325) (end 89.2 59.325) (width 0.5) (layer "B.Cu") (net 15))
 (segment (start 89.2 59.325) (end 89.15 59.375) (width 0.5) (layer "B.Cu") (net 15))
 (segment (start 44.704 63.246) (end 44.704 57.06) (width 0.5) (layer "B.Cu") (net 15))
 (segment (start 89.916 53.848) (end 89.408 53.34) (width 0.5) (layer "B.Cu") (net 15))
 (segment (start 84.179 63.246) (end 75.438 63.246) (width 0.5) (layer "B.Cu") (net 15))
 (segment (start 85.175 61.677082) (end 85.175 62.25) (width 0.5) (layer "B.Cu") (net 15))
 (segment (start 74.168 64.516) (end 45.974 64.516) (width 0.5) (layer "B.Cu") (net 15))
 (segment (start 85.598 60.452) (end 84.375 61.675) (width 0.5) (layer "F.Cu") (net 14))
 (segment (start 74.235 64.516) (end 75.438 63.313) (width 0.5) (layer "F.Cu") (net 14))
 (segment (start 86.6 59.325) (end 85.598 60.327) (width 0.25) (layer "F.Cu") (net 14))
 (segment (start 83.6 62.1) (end 84.025 61.675) (width 0.5) (layer "F.Cu") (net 14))
 (segment (start 76.651 62.1) (end 83.6 62.1) (width 0.5) (layer "F.Cu") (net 14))
 (segment (start 43.27 54.52) (end 42.926 54.864) (width 0.5) (layer "F.Cu") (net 14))
 (segment (start 42.926 54.864) (end 42.926 62.484) (width 0.5) (layer "F.Cu") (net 14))
 (segment (start 42.926 62.484) (end 44.958 64.516) (width 0.5) (layer "F.Cu") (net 14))
 (segment (start 44.704 54.52) (end 43.27 54.52) (width 0.5) (layer "F.Cu") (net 14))
 (segment (start 85.598 51.308) (end 85.09 50.8) (width 0.5) (layer "F.Cu") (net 14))
 (segment (start 75.438 63.313) (end 76.651 62.1) (width 0.5) (layer "F.Cu") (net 14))
 (segment (start 85.598 60.327) (end 85.598 60.452) (width 0.25) (layer "F.Cu") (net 14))
 (segment (start 44.958 64.516) (end 74.235 64.516) (width 0.5) (layer "F.Cu") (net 14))
 (segment (start 85.09 50.8) (end 85.09 47.498) (width 0.5) (layer "F.Cu") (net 14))
 (segment (start 85.598 60.452) (end 85.598 51.308) (width 0.5) (layer "F.Cu") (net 14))
 (segment (start 84.375 61.675) (end 84.025 61.675) (width 0.5) (layer "F.Cu") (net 14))
 (via (at 85.09 47.498) (size 0.8) (drill 0.4) (layers "F.Cu" "B.Cu") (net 14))
 (via (at 86.6 59.325) (size 0.8) (drill 0.4) (layers "F.Cu" "B.Cu") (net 14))
 (via (at 84.025 61.675) (size 0.8) (drill 0.4) (layers "F.Cu" "B.Cu") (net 14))
 (segment (start 85.598 45.974) (end 86.36 46.736) (width 0.5) (layer "F.Cu") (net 10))
 (segment (start 84.328 45.974) (end 85.598 45.974) (width 0.5) (layer "F.Cu") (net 10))
 (segment (start 83.566 46.736) (end 82.864 46.736) (width 0.5) (layer "F.Cu") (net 10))
 (segment (start 86.868 49.784) (end 91.71 49.784) (width 0.5) (layer "F.Cu") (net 10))
 (segment (start 84.328 45.974) (end 83.566 46.736) (width 0.5) (layer "F.Cu") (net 10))
 (segment (start 91.71 49.784) (end 91.8 49.874) (width 0.5) (layer "F.Cu") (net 10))
 (segment (start 86.36 46.736) (end 86.36 49.276) (width 0.5) (layer "F.Cu") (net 10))
 (segment (start 86.36 49.276) (end 86.868 49.784) (width 0.5) (layer "F.Cu") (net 10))
 (segment (start 44.704 42.418) (end 45.72 41.402) (width 0.25) (layer "F.Cu") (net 11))
 (segment (start 45.72 41.402) (end 81.788 41.402) (width 0.25) (layer "F.Cu") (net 11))
 (segment (start 82.55 42.164) (end 82.55 42.926) (width 0.25) (layer "F.Cu") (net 11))
 (segment (start 81.788 41.402) (end 82.55 42.164) (width 0.25) (layer "F.Cu") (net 11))
 (segment (start 44.704 46.9) (end 44.704 42.418) (width 0.25) (layer "F.Cu") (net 11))
 (via (at 82.55 42.926) (size 0.8) (drill 0.4) (layers "F.Cu" "B.Cu") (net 11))
 (segment (start 85.09 41.402) (end 85.09 42.926) (width 0.25) (layer "F.Cu") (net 12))
 (segment (start 74.734 40.952) (end 84.64 40.952) (width 0.25) (layer "F.Cu") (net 12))
 (segment (start 45.533604 40.952) (end 74.734 40.952) (width 0.25) (layer "F.Cu") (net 12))
 (segment (start 44.704 49.44) (end 43.852 49.44) (width 0.25) (layer "F.Cu") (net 12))
 (segment (start 42.926 43.559604) (end 45.533604 40.952) (width 0.25) (layer "F.Cu") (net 12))
 (segment (start 42.926 48.514) (end 42.926 43.559604) (width 0.25) (layer "F.Cu") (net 12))
 (segment (start 43.852 49.44) (end 42.926 48.514) (width 0.25) (layer "F.Cu") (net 12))
 (segment (start 84.64 40.952) (end 85.09 41.402) (width 0.25) (layer "F.Cu") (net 12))
 (via (at 85.09 42.926) (size 0.8) (drill 0.4) (layers "F.Cu" "B.Cu") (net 12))
 (segment (start 77.666 59.852396) (end 78.963604 61.15) (width 0.25) (layer "F.Cu") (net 4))
 (segment (start 78.963604 61.15) (end 83.265 61.15) (width 0.25) (layer "F.Cu") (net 4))
 (segment (start 83.265 61.15) (end 84.07 60.345) (width 0.25) (layer "F.Cu") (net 4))
 (segment (start 77.666 56.076) (end 77.666 59.15) (width 0.25) (layer "F.Cu") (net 4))
 (segment (start 76.11 54.52) (end 77.666 56.076) (width 0.25) (layer "F.Cu") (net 4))
 (segment (start 74.676 54.52) (end 76.11 54.52) (width 0.25) (layer "F.Cu") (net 4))
 (segment (start 77.666 59.15) (end 77.666 59.852396) (width 0.25) (layer "F.Cu") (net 4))
 (via (at 84.07 60.345) (size 0.8) (drill 0.4) (layers "F.Cu" "B.Cu") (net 4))
 (segment (start 84.07 59.375) (end 84.07 60.345) (width 0.25) (layer "B.Cu") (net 4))
 (segment (start 78.116 59.666) (end 78.745 60.295) (width 0.25) (layer "F.Cu") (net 3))
 (segment (start 78.116 58.925) (end 78.116 59.666) (width 0.25) (layer "F.Cu") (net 3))
 (segment (start 78.745 60.295) (end 81.53 60.295) (width 0.25) (layer "F.Cu") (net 3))
 (segment (start 74.676 51.98) (end 78.116 55.42) (width 0.25) (layer "F.Cu") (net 3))
 (segment (start 78.116 55.42) (end 78.116 58.925) (width 0.25) (layer "F.Cu") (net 3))
 (via (at 81.53 60.295) (size 0.8) (drill 0.4) (layers "F.Cu" "B.Cu") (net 3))
 (segment (start 81.53 59.375) (end 81.53 60.295) (width 0.25) (layer "B.Cu") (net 3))
 (segment (start 42.926 50.202) (end 42.926 42.418) (width 0.5) (layer "B.Cu") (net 13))
 (segment (start 42.926 42.418) (end 44.196 41.148) (width 0.5) (layer "B.Cu") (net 13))
 (segment (start 82.55 46.228) (end 82.55 47.468) (width 0.5) (layer "B.Cu") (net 13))
 (segment (start 82.042 45.72) (end 82.55 46.228) (width 0.5) (layer "B.Cu") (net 13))
 (segment (start 44.704 51.98) (end 42.926 50.202) (width 0.5) (layer "B.Cu") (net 13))
 (segment (start 79.248 45.72) (end 82.042 45.72) (width 0.5) (layer "B.Cu") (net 13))
 (segment (start 44.196 41.148) (end 74.676 41.148) (width 0.5) (layer "B.Cu") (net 13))
 (segment (start 74.676 41.148) (end 79.248 45.72) (width 0.5) (layer "B.Cu") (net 13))
 (segment (start 76.29 57.06) (end 76.962 56.388) (width 0.25) (layer "B.Cu") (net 5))
 (segment (start 76.962 49.022) (end 78.516 47.468) (width 0.25) (layer "B.Cu") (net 5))
 (segment (start 74.676 57.06) (end 76.29 57.06) (width 0.25) (layer "B.Cu") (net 5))
 (segment (start 78.516 47.468) (end 80.01 47.468) (width 0.25) (layer "B.Cu") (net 5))
 (segment (start 76.962 56.388) (end 76.962 49.022) (width 0.25) (layer "B.Cu") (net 5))
 (segment (start 81.534 48.768) (end 81.534 46.766) (width 0.5) (layer "F.Cu") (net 9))
 (segment (start 81.534 46.766) (end 81.564 46.736) (width 0.5) (layer "F.Cu") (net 9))
 (via (at 81.534 48.768) (size 0.8) (drill 0.4) (layers "F.Cu" "B.Cu") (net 9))
 (segment (start 80.01 48.768) (end 81.534 48.768) (width 0.5) (layer "B.Cu") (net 9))
 (segment (start 82.55 48.768) (end 85.09 48.768) (width 0.5) (layer "B.Cu") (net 9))
 (segment (start 81.534 48.768) (end 82.55 48.768) (width 0.5) (layer "B.Cu") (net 9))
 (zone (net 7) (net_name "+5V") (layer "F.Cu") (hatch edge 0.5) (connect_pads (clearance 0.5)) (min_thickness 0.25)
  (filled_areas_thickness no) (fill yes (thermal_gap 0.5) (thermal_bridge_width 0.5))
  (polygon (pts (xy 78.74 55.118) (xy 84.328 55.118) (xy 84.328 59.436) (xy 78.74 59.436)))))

